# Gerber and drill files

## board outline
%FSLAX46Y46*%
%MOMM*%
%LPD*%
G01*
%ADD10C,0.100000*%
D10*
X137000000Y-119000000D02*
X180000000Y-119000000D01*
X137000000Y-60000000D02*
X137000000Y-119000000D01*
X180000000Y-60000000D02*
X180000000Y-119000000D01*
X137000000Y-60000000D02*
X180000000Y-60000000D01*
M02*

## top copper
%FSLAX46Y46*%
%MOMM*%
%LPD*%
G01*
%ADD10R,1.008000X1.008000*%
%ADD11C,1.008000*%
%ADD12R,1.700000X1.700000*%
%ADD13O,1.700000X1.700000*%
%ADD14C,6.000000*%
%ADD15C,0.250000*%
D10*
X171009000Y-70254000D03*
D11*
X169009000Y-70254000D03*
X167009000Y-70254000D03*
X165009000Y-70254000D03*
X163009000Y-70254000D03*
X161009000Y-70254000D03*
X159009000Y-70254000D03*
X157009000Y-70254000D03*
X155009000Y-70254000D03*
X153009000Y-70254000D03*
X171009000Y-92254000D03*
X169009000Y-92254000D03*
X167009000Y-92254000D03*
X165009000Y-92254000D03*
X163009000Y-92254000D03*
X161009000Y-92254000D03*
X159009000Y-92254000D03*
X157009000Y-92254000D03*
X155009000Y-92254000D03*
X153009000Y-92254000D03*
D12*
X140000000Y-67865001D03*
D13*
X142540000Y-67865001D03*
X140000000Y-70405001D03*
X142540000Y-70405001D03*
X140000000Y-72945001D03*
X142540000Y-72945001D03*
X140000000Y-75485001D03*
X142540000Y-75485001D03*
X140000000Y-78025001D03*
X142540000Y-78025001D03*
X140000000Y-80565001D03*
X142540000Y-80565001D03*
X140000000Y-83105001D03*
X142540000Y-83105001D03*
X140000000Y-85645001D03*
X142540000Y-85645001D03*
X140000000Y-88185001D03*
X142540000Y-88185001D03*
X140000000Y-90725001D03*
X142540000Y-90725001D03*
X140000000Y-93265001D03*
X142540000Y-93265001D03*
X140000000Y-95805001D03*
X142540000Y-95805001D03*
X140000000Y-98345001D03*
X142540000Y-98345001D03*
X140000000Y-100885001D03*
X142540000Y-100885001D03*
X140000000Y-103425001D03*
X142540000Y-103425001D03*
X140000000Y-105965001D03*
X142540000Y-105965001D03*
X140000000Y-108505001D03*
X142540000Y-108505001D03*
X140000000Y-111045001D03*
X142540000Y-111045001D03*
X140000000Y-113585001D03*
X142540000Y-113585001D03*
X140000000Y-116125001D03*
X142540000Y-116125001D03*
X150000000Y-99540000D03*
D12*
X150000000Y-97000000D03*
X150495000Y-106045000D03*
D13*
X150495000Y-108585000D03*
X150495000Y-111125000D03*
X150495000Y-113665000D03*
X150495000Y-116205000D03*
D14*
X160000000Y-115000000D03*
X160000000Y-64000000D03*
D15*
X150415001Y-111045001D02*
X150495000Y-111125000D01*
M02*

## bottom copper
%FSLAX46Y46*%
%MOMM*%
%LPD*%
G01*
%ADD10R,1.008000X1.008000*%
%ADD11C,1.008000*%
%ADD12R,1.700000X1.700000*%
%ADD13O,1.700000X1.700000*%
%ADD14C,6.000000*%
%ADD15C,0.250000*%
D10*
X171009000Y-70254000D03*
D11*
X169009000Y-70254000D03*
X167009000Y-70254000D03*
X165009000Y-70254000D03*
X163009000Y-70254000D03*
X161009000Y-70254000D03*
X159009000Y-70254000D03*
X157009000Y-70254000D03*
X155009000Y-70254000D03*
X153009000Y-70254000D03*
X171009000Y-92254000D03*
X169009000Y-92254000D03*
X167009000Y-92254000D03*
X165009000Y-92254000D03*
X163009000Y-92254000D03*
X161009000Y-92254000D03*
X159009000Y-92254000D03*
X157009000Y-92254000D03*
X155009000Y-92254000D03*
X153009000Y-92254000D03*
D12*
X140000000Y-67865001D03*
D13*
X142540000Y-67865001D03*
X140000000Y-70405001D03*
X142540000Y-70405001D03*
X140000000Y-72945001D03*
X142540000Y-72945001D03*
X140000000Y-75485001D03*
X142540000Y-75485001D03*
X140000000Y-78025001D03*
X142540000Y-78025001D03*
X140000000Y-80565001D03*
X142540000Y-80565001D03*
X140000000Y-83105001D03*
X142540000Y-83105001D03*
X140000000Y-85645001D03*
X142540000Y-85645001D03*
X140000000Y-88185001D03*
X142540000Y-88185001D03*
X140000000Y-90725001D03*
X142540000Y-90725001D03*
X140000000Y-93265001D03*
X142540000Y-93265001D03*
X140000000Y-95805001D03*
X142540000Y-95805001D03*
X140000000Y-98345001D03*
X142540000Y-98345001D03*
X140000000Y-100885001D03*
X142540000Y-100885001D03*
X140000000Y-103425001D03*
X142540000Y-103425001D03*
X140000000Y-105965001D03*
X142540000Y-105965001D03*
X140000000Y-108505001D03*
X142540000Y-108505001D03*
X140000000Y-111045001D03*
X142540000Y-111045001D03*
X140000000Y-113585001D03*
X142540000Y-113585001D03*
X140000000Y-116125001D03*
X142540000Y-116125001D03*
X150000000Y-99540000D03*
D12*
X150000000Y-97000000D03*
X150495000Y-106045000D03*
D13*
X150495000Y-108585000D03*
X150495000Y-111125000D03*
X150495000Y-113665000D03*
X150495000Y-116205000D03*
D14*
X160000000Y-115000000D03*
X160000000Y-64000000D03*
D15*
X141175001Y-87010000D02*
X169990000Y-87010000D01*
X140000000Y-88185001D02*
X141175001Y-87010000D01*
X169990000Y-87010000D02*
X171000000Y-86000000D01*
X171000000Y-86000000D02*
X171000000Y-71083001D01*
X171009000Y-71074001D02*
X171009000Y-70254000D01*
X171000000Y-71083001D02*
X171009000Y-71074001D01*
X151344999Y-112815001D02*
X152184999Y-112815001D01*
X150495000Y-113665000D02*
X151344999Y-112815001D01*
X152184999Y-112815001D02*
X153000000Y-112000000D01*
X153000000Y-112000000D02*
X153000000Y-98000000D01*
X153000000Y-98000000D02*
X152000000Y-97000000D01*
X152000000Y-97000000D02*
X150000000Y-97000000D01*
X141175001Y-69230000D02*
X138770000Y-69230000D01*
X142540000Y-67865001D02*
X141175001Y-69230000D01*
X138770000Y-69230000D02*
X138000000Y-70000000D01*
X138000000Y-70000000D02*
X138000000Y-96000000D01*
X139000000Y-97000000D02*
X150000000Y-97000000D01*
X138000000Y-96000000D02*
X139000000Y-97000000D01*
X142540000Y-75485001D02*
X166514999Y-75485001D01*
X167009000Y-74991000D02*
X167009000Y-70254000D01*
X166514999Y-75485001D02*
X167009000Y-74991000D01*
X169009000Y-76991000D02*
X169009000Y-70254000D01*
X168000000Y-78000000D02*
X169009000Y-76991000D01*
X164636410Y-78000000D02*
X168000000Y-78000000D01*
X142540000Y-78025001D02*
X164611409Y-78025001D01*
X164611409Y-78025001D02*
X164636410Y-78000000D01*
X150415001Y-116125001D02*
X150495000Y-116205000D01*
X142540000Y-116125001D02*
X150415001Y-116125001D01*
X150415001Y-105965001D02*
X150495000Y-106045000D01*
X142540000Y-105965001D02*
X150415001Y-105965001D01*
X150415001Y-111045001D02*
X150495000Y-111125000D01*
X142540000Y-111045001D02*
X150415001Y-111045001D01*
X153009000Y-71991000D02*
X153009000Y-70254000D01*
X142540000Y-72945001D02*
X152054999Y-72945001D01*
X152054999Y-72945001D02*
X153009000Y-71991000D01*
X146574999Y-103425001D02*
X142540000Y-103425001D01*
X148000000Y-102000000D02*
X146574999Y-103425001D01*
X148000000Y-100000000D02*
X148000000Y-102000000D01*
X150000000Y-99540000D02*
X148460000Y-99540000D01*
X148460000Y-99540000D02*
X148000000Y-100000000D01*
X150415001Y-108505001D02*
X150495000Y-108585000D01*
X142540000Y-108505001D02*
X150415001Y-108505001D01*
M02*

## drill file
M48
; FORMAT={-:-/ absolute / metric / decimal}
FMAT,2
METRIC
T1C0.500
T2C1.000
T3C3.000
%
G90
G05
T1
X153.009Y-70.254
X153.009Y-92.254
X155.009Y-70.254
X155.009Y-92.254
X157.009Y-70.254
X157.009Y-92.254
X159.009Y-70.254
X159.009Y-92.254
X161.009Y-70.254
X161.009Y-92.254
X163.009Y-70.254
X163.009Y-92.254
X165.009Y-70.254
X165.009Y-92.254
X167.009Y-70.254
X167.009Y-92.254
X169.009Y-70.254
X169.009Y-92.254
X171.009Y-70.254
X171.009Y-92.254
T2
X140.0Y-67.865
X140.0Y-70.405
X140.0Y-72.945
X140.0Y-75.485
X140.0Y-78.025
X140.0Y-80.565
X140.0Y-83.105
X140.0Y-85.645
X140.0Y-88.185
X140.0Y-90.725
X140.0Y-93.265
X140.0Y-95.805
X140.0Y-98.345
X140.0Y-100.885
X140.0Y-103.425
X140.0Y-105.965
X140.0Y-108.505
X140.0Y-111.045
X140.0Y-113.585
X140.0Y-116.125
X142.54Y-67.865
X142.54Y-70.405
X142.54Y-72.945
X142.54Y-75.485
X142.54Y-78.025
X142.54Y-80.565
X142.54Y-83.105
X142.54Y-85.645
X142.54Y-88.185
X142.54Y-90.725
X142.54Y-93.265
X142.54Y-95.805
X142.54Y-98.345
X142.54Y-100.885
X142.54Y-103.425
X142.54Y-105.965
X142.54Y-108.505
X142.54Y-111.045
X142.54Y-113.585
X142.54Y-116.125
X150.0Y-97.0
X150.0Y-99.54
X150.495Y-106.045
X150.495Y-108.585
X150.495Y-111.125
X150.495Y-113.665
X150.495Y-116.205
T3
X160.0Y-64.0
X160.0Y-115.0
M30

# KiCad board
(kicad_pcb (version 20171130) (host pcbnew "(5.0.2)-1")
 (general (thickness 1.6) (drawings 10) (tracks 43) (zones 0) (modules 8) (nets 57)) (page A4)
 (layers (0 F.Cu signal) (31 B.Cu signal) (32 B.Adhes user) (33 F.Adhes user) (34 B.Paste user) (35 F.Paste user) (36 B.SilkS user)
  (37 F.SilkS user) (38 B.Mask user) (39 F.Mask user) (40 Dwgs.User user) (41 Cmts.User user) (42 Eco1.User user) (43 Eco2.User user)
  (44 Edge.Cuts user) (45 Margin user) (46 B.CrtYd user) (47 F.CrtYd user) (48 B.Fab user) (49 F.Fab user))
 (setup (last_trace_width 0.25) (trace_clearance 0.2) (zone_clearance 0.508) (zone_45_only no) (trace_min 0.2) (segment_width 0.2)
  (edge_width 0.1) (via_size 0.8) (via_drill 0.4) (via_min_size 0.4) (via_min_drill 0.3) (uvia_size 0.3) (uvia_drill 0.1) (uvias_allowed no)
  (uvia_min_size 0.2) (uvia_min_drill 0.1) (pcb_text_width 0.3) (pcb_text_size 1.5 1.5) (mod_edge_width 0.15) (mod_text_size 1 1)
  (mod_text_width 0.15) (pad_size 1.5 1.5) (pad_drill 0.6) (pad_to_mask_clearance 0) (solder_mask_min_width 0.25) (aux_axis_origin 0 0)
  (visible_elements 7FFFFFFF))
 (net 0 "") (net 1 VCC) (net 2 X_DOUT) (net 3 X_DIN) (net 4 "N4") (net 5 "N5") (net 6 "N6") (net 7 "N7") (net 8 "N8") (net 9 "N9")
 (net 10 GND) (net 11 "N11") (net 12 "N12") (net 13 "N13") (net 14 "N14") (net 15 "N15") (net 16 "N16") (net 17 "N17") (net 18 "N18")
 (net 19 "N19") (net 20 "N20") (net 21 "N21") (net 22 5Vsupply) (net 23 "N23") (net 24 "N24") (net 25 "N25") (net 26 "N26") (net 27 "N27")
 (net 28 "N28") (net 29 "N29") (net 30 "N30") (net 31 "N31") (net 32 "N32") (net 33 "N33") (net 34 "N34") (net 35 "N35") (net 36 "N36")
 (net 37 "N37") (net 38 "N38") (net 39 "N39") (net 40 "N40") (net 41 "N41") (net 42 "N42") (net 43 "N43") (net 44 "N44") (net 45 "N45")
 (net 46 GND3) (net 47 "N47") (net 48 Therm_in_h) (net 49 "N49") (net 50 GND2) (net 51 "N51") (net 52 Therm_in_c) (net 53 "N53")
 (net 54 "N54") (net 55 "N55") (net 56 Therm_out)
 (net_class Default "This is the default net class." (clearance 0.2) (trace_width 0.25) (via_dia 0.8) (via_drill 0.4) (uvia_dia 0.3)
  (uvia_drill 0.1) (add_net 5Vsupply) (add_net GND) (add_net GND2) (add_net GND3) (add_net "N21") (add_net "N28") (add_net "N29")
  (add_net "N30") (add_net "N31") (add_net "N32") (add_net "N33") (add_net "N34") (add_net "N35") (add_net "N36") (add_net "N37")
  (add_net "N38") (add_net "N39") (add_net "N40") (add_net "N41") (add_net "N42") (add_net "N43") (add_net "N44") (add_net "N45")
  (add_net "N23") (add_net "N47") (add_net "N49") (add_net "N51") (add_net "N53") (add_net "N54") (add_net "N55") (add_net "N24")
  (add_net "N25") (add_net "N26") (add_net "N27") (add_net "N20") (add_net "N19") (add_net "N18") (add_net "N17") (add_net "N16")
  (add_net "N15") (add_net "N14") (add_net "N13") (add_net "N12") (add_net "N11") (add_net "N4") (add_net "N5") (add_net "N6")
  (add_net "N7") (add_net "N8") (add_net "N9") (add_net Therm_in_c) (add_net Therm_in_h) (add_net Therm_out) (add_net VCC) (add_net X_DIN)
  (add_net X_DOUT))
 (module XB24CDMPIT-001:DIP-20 (layer F.Cu) (at 145 69 270)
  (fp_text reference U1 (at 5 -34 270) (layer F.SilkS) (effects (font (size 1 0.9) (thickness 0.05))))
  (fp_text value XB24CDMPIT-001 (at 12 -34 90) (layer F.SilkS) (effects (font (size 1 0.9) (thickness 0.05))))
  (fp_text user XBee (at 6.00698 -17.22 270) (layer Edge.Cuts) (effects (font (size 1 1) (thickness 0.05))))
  (pad 1 thru_hole rect (at 1.254 -26.009 270) (size 1.008 1.008) (drill 0.5) (layers *.Cu *.Mask) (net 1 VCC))
  (pad 2 thru_hole circle (at 1.254 -24.009 270) (size 1.008 1.008) (drill 0.5) (layers *.Cu *.Mask) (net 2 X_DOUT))
  (pad 3 thru_hole circle (at 1.254 -22.009 270) (size 1.008 1.008) (drill 0.5) (layers *.Cu *.Mask) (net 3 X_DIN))
  (pad 4 thru_hole circle (at 1.254 -20.009 270) (size 1.008 1.008) (drill 0.5) (layers *.Cu *.Mask) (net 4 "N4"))
  (pad 5 thru_hole circle (at 1.254 -18.009 270) (size 1.008 1.008) (drill 0.5) (layers *.Cu *.Mask) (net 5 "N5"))
  (pad 6 thru_hole circle (at 1.254 -16.009 270) (size 1.008 1.008) (drill 0.5) (layers *.Cu *.Mask) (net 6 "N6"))
  (pad 7 thru_hole circle (at 1.254 -14.009 270) (size 1.008 1.008) (drill 0.5) (layers *.Cu *.Mask) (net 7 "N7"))
  (pad 8 thru_hole circle (at 1.254 -12.009 270) (size 1.008 1.008) (drill 0.5) (layers *.Cu *.Mask) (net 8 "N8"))
  (pad 9 thru_hole circle (at 1.254 -10.009 270) (size 1.008 1.008) (drill 0.5) (layers *.Cu *.Mask) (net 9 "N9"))
  (pad 10 thru_hole circle (at 1.254 -8.009 270) (size 1.008 1.008) (drill 0.5) (layers *.Cu *.Mask) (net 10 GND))
  (pad 20 thru_hole circle (at 23.254 -26.009 270) (size 1.008 1.008) (drill 0.5) (layers *.Cu *.Mask) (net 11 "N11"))
  (pad 19 thru_hole circle (at 23.254 -24.009 270) (size 1.008 1.008) (drill 0.5) (layers *.Cu *.Mask) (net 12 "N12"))
  (pad 18 thru_hole circle (at 23.254 -22.009 270) (size 1.008 1.008) (drill 0.5) (layers *.Cu *.Mask) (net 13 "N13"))
  (pad 17 thru_hole circle (at 23.254 -20.009 270) (size 1.008 1.008) (drill 0.5) (layers *.Cu *.Mask) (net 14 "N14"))
  (pad 16 thru_hole circle (at 23.254 -18.009 270) (size 1.008 1.008) (drill 0.5) (layers *.Cu *.Mask) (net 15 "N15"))
  (pad 15 thru_hole circle (at 23.254 -16.009 270) (size 1.008 1.008) (drill 0.5) (layers *.Cu *.Mask) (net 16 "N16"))
  (pad 14 thru_hole circle (at 23.254 -14.009 270) (size 1.008 1.008) (drill 0.5) (layers *.Cu *.Mask) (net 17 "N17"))
  (pad 13 thru_hole circle (at 23.254 -12.009 270) (size 1.008 1.008) (drill 0.5) (layers *.Cu *.Mask) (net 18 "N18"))
  (pad 12 thru_hole circle (at 23.254 -10.009 270) (size 1.008 1.008) (drill 0.5) (layers *.Cu *.Mask) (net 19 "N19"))
  (pad 11 thru_hole circle (at 23.254 -8.009 270) (size 1.008 1.008) (drill 0.5) (layers *.Cu *.Mask) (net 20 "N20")))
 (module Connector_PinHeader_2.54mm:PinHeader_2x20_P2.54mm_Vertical (layer F.Cu) (at 140 67.865001)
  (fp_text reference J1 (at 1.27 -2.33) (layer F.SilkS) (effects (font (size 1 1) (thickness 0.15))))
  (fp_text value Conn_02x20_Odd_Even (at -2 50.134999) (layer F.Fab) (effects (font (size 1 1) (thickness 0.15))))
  (pad 1 thru_hole rect (at 0 0) (size 1.7 1.7) (drill 1) (layers *.Cu *.Mask) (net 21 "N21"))
  (pad 2 thru_hole oval (at 2.54 0) (size 1.7 1.7) (drill 1) (layers *.Cu *.Mask) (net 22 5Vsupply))
  (pad 3 thru_hole oval (at 0 2.54) (size 1.7 1.7) (drill 1) (layers *.Cu *.Mask) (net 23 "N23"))
  (pad 4 thru_hole oval (at 2.54 2.54) (size 1.7 1.7) (drill 1) (layers *.Cu *.Mask) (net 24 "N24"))
  (pad 5 thru_hole oval (at 0 5.08) (size 1.7 1.7) (drill 1) (layers *.Cu *.Mask) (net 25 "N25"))
  (pad 6 thru_hole oval (at 2.54 5.08) (size 1.7 1.7) (drill 1) (layers *.Cu *.Mask) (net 10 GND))
  (pad 7 thru_hole oval (at 0 7.62) (size 1.7 1.7) (drill 1) (layers *.Cu *.Mask) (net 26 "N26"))
  (pad 8 thru_hole oval (at 2.54 7.62) (size 1.7 1.7) (drill 1) (layers *.Cu *.Mask) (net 3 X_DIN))
  (pad 9 thru_hole oval (at 0 10.16) (size 1.7 1.7) (drill 1) (layers *.Cu *.Mask) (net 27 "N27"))
  (pad 10 thru_hole oval (at 2.54 10.16) (size 1.7 1.7) (drill 1) (layers *.Cu *.Mask) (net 2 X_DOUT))
  (pad 11 thru_hole oval (at 0 12.7) (size 1.7 1.7) (drill 1) (layers *.Cu *.Mask) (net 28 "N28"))
  (pad 12 thru_hole oval (at 2.54 12.7) (size 1.7 1.7) (drill 1) (layers *.Cu *.Mask) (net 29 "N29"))
  (pad 13 thru_hole oval (at 0 15.24) (size 1.7 1.7) (drill 1) (layers *.Cu *.Mask) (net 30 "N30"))
  (pad 14 thru_hole oval (at 2.54 15.24) (size 1.7 1.7) (drill 1) (layers *.Cu *.Mask) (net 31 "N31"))
  (pad 15 thru_hole oval (at 0 17.78) (size 1.7 1.7) (drill 1) (layers *.Cu *.Mask) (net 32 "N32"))
  (pad 16 thru_hole oval (at 2.54 17.78) (size 1.7 1.7) (drill 1) (layers *.Cu *.Mask) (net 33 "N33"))
  (pad 17 thru_hole oval (at 0 20.32) (size 1.7 1.7) (drill 1) (layers *.Cu *.Mask) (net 1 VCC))
  (pad 18 thru_hole oval (at 2.54 20.32) (size 1.7 1.7) (drill 1) (layers *.Cu *.Mask) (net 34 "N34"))
  (pad 19 thru_hole oval (at 0 22.86) (size 1.7 1.7) (drill 1) (layers *.Cu *.Mask) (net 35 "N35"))
  (pad 20 thru_hole oval (at 2.54 22.86) (size 1.7 1.7) (drill 1) (layers *.Cu *.Mask) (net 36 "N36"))
  (pad 21 thru_hole oval (at 0 25.4) (size 1.7 1.7) (drill 1) (layers *.Cu *.Mask) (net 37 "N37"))
  (pad 22 thru_hole oval (at 2.54 25.4) (size 1.7 1.7) (drill 1) (layers *.Cu *.Mask) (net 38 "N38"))
  (pad 23 thru_hole oval (at 0 27.94) (size 1.7 1.7) (drill 1) (layers *.Cu *.Mask) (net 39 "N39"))
  (pad 24 thru_hole oval (at 2.54 27.94) (size 1.7 1.7) (drill 1) (layers *.Cu *.Mask) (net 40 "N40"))
  (pad 25 thru_hole oval (at 0 30.48) (size 1.7 1.7) (drill 1) (layers *.Cu *.Mask) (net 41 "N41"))
  (pad 26 thru_hole oval (at 2.54 30.48) (size 1.7 1.7) (drill 1) (layers *.Cu *.Mask) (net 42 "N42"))
  (pad 27 thru_hole oval (at 0 33.02) (size 1.7 1.7) (drill 1) (layers *.Cu *.Mask) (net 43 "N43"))
  (pad 28 thru_hole oval (at 2.54 33.02) (size 1.7 1.7) (drill 1) (layers *.Cu *.Mask) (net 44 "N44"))
  (pad 29 thru_hole oval (at 0 35.56) (size 1.7 1.7) (drill 1) (layers *.Cu *.Mask) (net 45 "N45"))
  (pad 30 thru_hole oval (at 2.54 35.56) (size 1.7 1.7) (drill 1) (layers *.Cu *.Mask) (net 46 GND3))
  (pad 31 thru_hole oval (at 0 38.1) (size 1.7 1.7) (drill 1) (layers *.Cu *.Mask) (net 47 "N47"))
  (pad 32 thru_hole oval (at 2.54 38.1) (size 1.7 1.7) (drill 1) (layers *.Cu *.Mask) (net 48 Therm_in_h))
  (pad 33 thru_hole oval (at 0 40.64) (size 1.7 1.7) (drill 1) (layers *.Cu *.Mask) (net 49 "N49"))
  (pad 34 thru_hole oval (at 2.54 40.64) (size 1.7 1.7) (drill 1) (layers *.Cu *.Mask) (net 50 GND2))
  (pad 35 thru_hole oval (at 0 43.18) (size 1.7 1.7) (drill 1) (layers *.Cu *.Mask) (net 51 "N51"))
  (pad 36 thru_hole oval (at 2.54 43.18) (size 1.7 1.7) (drill 1) (layers *.Cu *.Mask) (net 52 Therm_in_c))
  (pad 37 thru_hole oval (at 0 45.72) (size 1.7 1.7) (drill 1) (layers *.Cu *.Mask) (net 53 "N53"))
  (pad 38 thru_hole oval (at 2.54 45.72) (size 1.7 1.7) (drill 1) (layers *.Cu *.Mask) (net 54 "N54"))
  (pad 39 thru_hole oval (at 0 48.26) (size 1.7 1.7) (drill 1) (layers *.Cu *.Mask) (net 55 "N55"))
  (pad 40 thru_hole oval (at 2.54 48.26) (size 1.7 1.7) (drill 1) (layers *.Cu *.Mask) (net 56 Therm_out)))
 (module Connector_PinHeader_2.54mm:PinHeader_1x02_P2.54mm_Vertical (layer F.Cu) (at 150 97)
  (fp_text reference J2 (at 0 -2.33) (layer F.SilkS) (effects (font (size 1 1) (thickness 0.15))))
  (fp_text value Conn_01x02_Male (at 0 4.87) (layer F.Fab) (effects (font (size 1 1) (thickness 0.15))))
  (pad 2 thru_hole oval (at 0 2.54) (size 1.7 1.7) (drill 1) (layers *.Cu *.Mask) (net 46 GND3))
  (pad 1 thru_hole rect (at 0 0) (size 1.7 1.7) (drill 1) (layers *.Cu *.Mask) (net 22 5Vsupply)))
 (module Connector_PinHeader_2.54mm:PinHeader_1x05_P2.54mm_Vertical (layer F.Cu) (at 150.495 106.045)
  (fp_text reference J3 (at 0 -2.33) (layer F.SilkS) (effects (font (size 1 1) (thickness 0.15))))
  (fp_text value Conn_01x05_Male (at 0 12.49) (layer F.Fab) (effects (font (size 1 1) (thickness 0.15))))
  (pad 1 thru_hole rect (at 0 0) (size 1.7 1.7) (drill 1) (layers *.Cu *.Mask) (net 48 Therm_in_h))
  (pad 2 thru_hole oval (at 0 2.54) (size 1.7 1.7) (drill 1) (layers *.Cu *.Mask) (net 50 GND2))
  (pad 3 thru_hole oval (at 0 5.08) (size 1.7 1.7) (drill 1) (layers *.Cu *.Mask) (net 52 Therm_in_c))
  (pad 4 thru_hole oval (at 0 7.62) (size 1.7 1.7) (drill 1) (layers *.Cu *.Mask) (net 22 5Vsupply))
  (pad 5 thru_hole oval (at 0 10.16) (size 1.7 1.7) (drill 1) (layers *.Cu *.Mask) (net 56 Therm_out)))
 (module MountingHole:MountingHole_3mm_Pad (layer F.Cu) (at 160 115)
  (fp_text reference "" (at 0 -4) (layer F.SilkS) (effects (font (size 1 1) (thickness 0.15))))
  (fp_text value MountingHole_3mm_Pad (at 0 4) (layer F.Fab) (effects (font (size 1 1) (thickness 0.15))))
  (pad 1 thru_hole circle (at 0 0) (size 6 6) (drill 3) (layers *.Cu *.Mask)))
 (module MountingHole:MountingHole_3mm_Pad (layer F.Cu) (at 160 64)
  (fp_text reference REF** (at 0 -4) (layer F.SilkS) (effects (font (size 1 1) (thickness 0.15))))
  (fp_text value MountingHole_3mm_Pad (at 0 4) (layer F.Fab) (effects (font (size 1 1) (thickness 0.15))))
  (pad 1 thru_hole circle (at 0 0) (size 6 6) (drill 3) (layers *.Cu *.Mask)))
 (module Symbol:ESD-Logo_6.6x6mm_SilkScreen (layer F.Cu) (at 175 114)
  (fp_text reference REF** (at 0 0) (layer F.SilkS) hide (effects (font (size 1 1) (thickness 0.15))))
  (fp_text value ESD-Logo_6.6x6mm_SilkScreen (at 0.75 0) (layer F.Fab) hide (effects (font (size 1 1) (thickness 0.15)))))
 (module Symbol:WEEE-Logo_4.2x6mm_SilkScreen (layer F.Cu) (at 168 114)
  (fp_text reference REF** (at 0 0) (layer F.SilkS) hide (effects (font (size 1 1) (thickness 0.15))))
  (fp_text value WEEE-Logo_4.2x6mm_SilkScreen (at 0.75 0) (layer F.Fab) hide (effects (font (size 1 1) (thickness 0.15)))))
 (gr_line (start 137 119) (end 180 119) (layer Edge.Cuts) (width 0.1))
 (gr_line (start 137 60) (end 137 119) (layer Edge.Cuts) (width 0.1))
 (gr_line (start 180 60) (end 180 119) (layer Edge.Cuts) (width 0.1))
 (gr_line (start 137 60) (end 180 60) (layer Edge.Cuts) (width 0.1))
 (segment (start 141.175001 87.01) (end 169.99 87.01) (width 0.25) (layer B.Cu) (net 1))
 (segment (start 140 88.185001) (end 141.175001 87.01) (width 0.25) (layer B.Cu) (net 1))
 (segment (start 169.99 87.01) (end 171 86) (width 0.25) (layer B.Cu) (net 1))
 (segment (start 171 86) (end 171 71.083001) (width 0.25) (layer B.Cu) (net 1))
 (segment (start 171.009 71.074001) (end 171.009 70.254) (width 0.25) (layer B.Cu) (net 1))
 (segment (start 171 71.083001) (end 171.009 71.074001) (width 0.25) (layer B.Cu) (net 1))
 (segment (start 151.344999 112.815001) (end 152.184999 112.815001) (width 0.25) (layer B.Cu) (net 22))
 (segment (start 150.495 113.665) (end 151.344999 112.815001) (width 0.25) (layer B.Cu) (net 22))
 (segment (start 152.184999 112.815001) (end 153 112) (width 0.25) (layer B.Cu) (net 22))
 (segment (start 153 112) (end 153 98) (width 0.25) (layer B.Cu) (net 22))
 (segment (start 153 98) (end 152 97) (width 0.25) (layer B.Cu) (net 22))
 (segment (start 152 97) (end 150 97) (width 0.25) (layer B.Cu) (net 22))
 (segment (start 141.175001 69.23) (end 138.77 69.23) (width 0.25) (layer B.Cu) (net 22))
 (segment (start 142.54 67.865001) (end 141.175001 69.23) (width 0.25) (layer B.Cu) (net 22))
 (segment (start 138.77 69.23) (end 138 70) (width 0.25) (layer B.Cu) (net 22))
 (segment (start 138 70) (end 138 96) (width 0.25) (layer B.Cu) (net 22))
 (segment (start 139 97) (end 150 97) (width 0.25) (layer B.Cu) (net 22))
 (segment (start 138 96) (end 139 97) (width 0.25) (layer B.Cu) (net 22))
 (segment (start 142.54 75.485001) (end 166.514999 75.485001) (width 0.25) (layer B.Cu) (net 3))
 (segment (start 167.009 74.991) (end 167.009 70.254) (width 0.25) (layer B.Cu) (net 3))
 (segment (start 166.514999 75.485001) (end 167.009 74.991) (width 0.25) (layer B.Cu) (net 3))
 (segment (start 169.009 76.991) (end 169.009 70.254) (width 0.25) (layer B.Cu) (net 2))
 (segment (start 168 78) (end 169.009 76.991) (width 0.25) (layer B.Cu) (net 2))
 (segment (start 164.63641 78) (end 168 78) (width 0.25) (layer B.Cu) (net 2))
 (segment (start 142.54 78.025001) (end 164.611409 78.025001) (width 0.25) (layer B.Cu) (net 2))
 (segment (start 164.611409 78.025001) (end 164.63641 78) (width 0.25) (layer B.Cu) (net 2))
 (segment (start 150.415001 116.125001) (end 150.495 116.205) (width 0.25) (layer B.Cu) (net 56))
 (segment (start 142.54 116.125001) (end 150.415001 116.125001) (width 0.25) (layer B.Cu) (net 56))
 (segment (start 150.415001 105.965001) (end 150.495 106.045) (width 0.25) (layer B.Cu) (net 48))
 (segment (start 142.54 105.965001) (end 150.415001 105.965001) (width 0.25) (layer B.Cu) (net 48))
 (segment (start 150.415001 111.045001) (end 150.495 111.125) (width 0.25) (layer F.Cu) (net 52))
 (segment (start 150.415001 111.045001) (end 150.495 111.125) (width 0.25) (layer B.Cu) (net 52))
 (segment (start 142.54 111.045001) (end 150.415001 111.045001) (width 0.25) (layer B.Cu) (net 52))
 (segment (start 153.009 71.991) (end 153.009 70.254) (width 0.25) (layer B.Cu) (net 10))
 (segment (start 142.54 72.945001) (end 152.054999 72.945001) (width 0.25) (layer B.Cu) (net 10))
 (segment (start 152.054999 72.945001) (end 153.009 71.991) (width 0.25) (layer B.Cu) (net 10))
 (segment (start 146.574999 103.425001) (end 142.54 103.425001) (width 0.25) (layer B.Cu) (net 46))
 (segment (start 148 102) (end 146.574999 103.425001) (width 0.25) (layer B.Cu) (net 46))
 (segment (start 148 100) (end 148 102) (width 0.25) (layer B.Cu) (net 46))
 (segment (start 150 99.54) (end 148.46 99.54) (width 0.25) (layer B.Cu) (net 46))
 (segment (start 148.46 99.54) (end 148 100) (width 0.25) (layer B.Cu) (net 46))
 (segment (start 150.415001 108.505001) (end 150.495 108.585) (width 0.25) (layer B.Cu) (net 50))
 (segment (start 142.54 108.505001) (end 150.415001 108.505001) (width 0.25) (layer B.Cu) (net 50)))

